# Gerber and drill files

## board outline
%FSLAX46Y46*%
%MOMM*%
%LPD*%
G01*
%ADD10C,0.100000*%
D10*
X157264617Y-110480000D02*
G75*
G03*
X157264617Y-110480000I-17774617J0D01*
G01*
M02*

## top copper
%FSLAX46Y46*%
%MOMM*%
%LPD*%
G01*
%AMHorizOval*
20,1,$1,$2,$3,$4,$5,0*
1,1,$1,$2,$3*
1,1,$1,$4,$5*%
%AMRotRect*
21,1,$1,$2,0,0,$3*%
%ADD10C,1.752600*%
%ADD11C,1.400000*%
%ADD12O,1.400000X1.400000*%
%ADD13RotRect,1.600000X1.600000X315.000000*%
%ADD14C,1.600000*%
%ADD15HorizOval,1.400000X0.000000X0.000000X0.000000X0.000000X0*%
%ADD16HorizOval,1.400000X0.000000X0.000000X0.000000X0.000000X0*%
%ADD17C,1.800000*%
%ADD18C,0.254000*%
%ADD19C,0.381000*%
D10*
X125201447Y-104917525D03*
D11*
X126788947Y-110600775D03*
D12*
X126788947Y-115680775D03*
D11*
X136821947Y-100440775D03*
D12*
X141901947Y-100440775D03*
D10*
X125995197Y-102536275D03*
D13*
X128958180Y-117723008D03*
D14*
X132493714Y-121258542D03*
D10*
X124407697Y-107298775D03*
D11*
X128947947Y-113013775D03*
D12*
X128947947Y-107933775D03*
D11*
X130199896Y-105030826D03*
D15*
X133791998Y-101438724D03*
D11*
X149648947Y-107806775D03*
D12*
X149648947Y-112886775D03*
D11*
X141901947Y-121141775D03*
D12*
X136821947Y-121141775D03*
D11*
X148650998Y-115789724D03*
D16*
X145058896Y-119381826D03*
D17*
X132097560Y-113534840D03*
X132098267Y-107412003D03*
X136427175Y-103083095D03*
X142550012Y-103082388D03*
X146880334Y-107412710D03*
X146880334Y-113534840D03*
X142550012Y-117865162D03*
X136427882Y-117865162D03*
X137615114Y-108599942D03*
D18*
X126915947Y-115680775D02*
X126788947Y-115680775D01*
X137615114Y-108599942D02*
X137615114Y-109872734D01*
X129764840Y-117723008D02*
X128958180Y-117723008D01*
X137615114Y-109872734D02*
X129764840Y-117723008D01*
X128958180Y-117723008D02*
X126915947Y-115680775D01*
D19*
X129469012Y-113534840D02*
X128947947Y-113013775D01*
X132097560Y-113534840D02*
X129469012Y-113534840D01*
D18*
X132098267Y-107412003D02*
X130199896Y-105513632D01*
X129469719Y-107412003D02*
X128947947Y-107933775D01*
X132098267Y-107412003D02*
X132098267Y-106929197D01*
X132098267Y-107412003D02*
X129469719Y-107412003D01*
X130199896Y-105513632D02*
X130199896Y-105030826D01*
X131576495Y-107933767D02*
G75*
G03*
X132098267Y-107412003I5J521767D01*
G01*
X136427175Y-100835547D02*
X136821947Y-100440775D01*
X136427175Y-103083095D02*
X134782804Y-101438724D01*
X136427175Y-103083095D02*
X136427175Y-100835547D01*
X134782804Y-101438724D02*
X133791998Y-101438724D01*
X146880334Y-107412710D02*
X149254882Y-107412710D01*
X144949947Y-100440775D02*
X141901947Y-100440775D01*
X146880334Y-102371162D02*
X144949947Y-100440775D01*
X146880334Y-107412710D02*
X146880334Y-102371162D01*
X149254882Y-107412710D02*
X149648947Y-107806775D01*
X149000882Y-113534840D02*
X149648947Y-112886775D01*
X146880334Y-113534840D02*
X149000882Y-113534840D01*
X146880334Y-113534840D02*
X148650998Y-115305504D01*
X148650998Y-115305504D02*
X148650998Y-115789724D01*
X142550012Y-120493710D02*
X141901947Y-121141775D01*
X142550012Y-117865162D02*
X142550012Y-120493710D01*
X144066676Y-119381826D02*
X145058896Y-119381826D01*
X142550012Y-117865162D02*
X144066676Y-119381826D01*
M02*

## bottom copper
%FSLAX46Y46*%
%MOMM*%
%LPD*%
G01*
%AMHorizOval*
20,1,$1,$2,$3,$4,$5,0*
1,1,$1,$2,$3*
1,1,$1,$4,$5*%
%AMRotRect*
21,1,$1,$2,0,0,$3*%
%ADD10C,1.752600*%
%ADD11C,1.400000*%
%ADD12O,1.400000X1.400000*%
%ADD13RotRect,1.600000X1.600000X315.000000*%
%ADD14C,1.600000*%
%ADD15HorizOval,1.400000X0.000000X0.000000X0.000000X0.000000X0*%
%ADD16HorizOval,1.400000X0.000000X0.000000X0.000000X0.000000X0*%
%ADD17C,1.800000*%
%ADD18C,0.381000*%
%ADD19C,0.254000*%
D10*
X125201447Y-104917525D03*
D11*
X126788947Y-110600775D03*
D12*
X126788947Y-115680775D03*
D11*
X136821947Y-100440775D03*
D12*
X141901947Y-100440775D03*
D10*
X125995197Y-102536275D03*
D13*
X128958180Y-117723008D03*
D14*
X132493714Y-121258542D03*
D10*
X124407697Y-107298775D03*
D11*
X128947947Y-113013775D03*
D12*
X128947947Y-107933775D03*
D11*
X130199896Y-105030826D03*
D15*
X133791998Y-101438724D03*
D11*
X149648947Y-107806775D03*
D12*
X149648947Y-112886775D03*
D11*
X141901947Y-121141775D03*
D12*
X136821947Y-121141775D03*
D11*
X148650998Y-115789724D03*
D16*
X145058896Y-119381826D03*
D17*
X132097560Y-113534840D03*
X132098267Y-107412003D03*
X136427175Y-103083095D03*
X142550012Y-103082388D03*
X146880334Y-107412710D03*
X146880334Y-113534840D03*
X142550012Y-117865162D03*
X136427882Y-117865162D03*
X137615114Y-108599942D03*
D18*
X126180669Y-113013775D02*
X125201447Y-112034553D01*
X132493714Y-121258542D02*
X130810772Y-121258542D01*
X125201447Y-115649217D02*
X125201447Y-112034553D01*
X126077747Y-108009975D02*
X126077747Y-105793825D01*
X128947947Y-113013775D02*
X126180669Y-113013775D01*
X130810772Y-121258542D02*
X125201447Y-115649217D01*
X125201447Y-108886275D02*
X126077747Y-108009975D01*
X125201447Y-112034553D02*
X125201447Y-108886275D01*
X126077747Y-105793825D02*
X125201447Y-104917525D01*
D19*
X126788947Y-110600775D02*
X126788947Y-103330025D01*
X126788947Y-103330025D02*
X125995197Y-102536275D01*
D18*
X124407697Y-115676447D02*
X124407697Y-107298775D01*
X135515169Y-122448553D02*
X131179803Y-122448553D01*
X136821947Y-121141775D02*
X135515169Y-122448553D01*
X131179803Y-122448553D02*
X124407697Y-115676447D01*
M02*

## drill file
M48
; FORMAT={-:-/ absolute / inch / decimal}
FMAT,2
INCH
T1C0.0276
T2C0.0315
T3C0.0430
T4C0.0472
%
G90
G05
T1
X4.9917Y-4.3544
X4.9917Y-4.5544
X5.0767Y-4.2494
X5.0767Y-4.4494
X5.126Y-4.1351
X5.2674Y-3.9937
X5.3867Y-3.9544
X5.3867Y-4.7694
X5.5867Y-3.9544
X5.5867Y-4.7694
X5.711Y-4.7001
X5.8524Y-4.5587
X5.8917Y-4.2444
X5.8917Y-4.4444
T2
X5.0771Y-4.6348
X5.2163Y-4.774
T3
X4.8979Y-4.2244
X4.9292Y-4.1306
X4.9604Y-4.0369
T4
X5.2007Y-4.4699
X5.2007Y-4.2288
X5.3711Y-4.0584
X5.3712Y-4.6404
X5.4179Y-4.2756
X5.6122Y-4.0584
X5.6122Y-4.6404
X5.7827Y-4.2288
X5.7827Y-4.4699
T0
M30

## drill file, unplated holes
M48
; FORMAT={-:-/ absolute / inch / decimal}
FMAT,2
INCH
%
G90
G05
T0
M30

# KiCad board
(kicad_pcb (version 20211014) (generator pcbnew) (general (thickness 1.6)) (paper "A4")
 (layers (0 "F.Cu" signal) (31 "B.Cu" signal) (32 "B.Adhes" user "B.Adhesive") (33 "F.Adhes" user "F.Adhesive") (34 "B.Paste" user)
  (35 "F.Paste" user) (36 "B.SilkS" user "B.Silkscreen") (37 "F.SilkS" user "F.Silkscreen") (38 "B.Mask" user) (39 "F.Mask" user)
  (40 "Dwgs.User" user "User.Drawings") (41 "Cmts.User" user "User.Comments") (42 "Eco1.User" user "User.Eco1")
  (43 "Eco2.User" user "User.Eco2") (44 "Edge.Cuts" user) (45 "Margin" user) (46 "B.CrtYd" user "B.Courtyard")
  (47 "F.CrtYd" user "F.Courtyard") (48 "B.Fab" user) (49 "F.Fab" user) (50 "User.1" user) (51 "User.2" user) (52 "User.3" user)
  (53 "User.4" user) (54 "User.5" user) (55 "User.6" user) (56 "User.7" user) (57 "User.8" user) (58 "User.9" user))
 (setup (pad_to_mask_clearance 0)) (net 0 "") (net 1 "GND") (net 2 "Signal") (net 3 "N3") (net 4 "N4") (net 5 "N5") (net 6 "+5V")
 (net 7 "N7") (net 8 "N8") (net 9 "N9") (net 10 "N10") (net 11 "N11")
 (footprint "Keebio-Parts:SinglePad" (layer "F.Cu") (at 125.201447 104.917525)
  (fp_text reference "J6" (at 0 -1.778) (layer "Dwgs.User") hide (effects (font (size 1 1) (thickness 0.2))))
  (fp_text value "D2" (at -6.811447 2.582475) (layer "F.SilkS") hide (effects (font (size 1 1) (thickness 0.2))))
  (pad "1" thru_hole circle locked (at 0 0 270) (size 1.7526 1.7526) (drill 1.0922) (layers *.Cu *.SilkS *.Mask) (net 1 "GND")))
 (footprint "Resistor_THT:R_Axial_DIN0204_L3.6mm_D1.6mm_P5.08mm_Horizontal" (layer "F.Cu") (at 126.788947 110.600775 -90)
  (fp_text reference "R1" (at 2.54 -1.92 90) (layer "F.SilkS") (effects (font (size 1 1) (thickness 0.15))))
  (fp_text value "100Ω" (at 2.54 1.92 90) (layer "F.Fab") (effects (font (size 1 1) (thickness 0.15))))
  (pad "1" thru_hole circle (at 0 0 270) (size 1.4 1.4) (drill 0.7) (layers *.Cu *.Mask) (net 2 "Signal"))
  (pad "2" thru_hole oval (at 5.08 0 270) (size 1.4 1.4) (drill 0.7) (layers *.Cu *.Mask) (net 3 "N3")))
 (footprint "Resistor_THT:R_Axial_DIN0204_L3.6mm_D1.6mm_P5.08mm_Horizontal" (layer "F.Cu") (at 136.821947 100.440775)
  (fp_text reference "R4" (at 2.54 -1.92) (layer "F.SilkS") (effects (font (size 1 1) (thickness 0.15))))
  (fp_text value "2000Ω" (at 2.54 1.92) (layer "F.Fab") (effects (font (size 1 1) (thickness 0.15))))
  (pad "1" thru_hole circle (at 0 0) (size 1.4 1.4) (drill 0.7) (layers *.Cu *.Mask) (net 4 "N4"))
  (pad "2" thru_hole oval (at 5.08 0) (size 1.4 1.4) (drill 0.7) (layers *.Cu *.Mask) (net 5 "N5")))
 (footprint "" (layer "F.Cu") (at 125.995197 102.536275)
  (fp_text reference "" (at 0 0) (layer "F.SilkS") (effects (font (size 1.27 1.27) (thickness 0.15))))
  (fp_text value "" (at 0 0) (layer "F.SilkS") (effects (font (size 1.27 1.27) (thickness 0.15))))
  (pad "1" thru_hole circle locked (at 0 0 270) (size 1.7526 1.7526) (drill 1.0922) (layers *.Cu *.SilkS *.Mask) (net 2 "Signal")))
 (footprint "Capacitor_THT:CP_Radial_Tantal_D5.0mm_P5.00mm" (layer "F.Cu") (at 128.95818 117.723008 -45)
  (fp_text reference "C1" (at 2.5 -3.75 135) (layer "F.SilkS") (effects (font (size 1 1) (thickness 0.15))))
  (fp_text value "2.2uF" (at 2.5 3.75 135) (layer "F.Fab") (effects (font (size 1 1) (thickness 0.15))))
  (pad "1" thru_hole rect (at 0 0 315) (size 1.6 1.6) (drill 0.8) (layers *.Cu *.Mask) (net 3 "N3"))
  (pad "2" thru_hole circle (at 5 0 315) (size 1.6 1.6) (drill 0.8) (layers *.Cu *.Mask) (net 1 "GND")))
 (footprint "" (layer "F.Cu") (at 124.407697 107.298775)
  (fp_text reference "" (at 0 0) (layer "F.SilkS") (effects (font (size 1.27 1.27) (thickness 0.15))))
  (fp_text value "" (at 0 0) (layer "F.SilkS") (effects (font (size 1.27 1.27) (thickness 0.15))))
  (pad "1" thru_hole circle locked (at 0 0 270) (size 1.7526 1.7526) (drill 1.0922) (layers *.Cu *.SilkS *.Mask) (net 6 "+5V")))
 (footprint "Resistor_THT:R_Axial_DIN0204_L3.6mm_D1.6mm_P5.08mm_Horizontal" (layer "F.Cu") (at 128.947947 113.013775 90)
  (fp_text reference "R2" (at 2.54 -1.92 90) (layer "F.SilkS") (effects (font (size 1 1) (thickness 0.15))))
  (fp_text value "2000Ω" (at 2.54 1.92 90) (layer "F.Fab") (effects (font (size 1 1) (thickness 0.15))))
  (pad "1" thru_hole circle (at 0 0 90) (size 1.4 1.4) (drill 0.7) (layers *.Cu *.Mask) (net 1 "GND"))
  (pad "2" thru_hole oval (at 5.08 0 90) (size 1.4 1.4) (drill 0.7) (layers *.Cu *.Mask) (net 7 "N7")))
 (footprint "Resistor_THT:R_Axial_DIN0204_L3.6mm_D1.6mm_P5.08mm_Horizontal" (layer "F.Cu") (at 130.199896 105.030826 45)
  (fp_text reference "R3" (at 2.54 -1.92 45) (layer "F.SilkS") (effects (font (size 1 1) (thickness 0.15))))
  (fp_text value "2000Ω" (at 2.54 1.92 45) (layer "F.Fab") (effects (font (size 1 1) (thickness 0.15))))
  (pad "1" thru_hole circle (at 0 0 45) (size 1.4 1.4) (drill 0.7) (layers *.Cu *.Mask) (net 7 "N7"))
  (pad "2" thru_hole oval (at 5.08 0 45) (size 1.4 1.4) (drill 0.7) (layers *.Cu *.Mask) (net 4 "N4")))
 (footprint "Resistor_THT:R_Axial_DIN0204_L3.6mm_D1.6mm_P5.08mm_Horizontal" (layer "F.Cu") (at 149.648947 107.806775 -90)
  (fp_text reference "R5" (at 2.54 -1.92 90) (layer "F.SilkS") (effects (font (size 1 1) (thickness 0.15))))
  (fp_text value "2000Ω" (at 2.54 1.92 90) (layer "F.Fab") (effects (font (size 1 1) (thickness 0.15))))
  (pad "1" thru_hole circle (at 0 0 270) (size 1.4 1.4) (drill 0.7) (layers *.Cu *.Mask) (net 5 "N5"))
  (pad "2" thru_hole oval (at 5.08 0 270) (size 1.4 1.4) (drill 0.7) (layers *.Cu *.Mask) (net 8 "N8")))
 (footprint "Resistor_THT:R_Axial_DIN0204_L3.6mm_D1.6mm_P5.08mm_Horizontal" (layer "F.Cu") (at 141.901947 121.141775 180)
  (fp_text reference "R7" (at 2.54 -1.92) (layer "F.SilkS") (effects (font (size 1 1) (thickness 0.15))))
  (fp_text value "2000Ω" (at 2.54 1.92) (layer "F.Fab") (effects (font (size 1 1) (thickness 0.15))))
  (pad "1" thru_hole circle (at 0 0 180) (size 1.4 1.4) (drill 0.7) (layers *.Cu *.Mask) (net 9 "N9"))
  (pad "2" thru_hole oval (at 5.08 0 180) (size 1.4 1.4) (drill 0.7) (layers *.Cu *.Mask) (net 6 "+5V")))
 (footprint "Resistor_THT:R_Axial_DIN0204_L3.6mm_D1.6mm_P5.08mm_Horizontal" (layer "F.Cu") (at 148.650998 115.789724 -135)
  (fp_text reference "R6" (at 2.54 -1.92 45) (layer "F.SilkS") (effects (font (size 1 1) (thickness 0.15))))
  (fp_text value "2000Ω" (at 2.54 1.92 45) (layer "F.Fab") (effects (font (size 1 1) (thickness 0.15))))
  (pad "1" thru_hole circle (at 0 0 225) (size 1.4 1.4) (drill 0.7) (layers *.Cu *.Mask) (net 8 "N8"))
  (pad "2" thru_hole oval (at 5.08 0 225) (size 1.4 1.4) (drill 0.7) (layers *.Cu *.Mask) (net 9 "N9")))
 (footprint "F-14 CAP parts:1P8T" (layer "B.Cu") (at 139.488947 110.473775 135)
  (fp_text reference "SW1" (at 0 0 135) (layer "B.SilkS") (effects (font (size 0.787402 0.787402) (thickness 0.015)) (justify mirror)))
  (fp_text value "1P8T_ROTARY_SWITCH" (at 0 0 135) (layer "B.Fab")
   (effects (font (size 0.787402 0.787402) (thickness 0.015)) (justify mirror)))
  (pad "1" thru_hole circle (at 3.062 -7.391 135) (size 1.8 1.8) (drill 1.2) (layers *.Cu *.Mask) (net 1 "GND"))
  (pad "2" thru_hole circle (at 7.391 -3.061 135) (size 1.8 1.8) (drill 1.2) (layers *.Cu *.Mask) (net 7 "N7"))
  (pad "3" thru_hole circle (at 7.391 3.061 135) (size 1.8 1.8) (drill 1.2) (layers *.Cu *.Mask) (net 4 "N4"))
  (pad "4" thru_hole circle (at 3.062 7.391 135) (size 1.8 1.8) (drill 1.2) (layers *.Cu *.Mask) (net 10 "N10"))
  (pad "5" thru_hole circle (at -3.062 7.391 135) (size 1.8 1.8) (drill 1.2) (layers *.Cu *.Mask) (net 5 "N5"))
  (pad "6" thru_hole circle (at -7.391 3.062 135) (size 1.8 1.8) (drill 1.2) (layers *.Cu *.Mask) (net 8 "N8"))
  (pad "7" thru_hole circle (at -7.391 -3.062 135) (size 1.8 1.8) (drill 1.2) (layers *.Cu *.Mask) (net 9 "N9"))
  (pad "8" thru_hole circle (at -3.062 -7.391 135) (size 1.8 1.8) (drill 1.2) (layers *.Cu *.Mask) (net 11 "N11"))
  (pad "9" thru_hole circle (at 2.65 0 135) (size 1.8 1.8) (drill 1.2) (layers *.Cu *.Mask) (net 3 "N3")))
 (gr_circle (center 139.49 110.48) (end 146.32 94.07) (layer "Edge.Cuts") (width 0.1) (fill none))
 (segment (start 126.915947 115.680775) (end 126.788947 115.680775) (width 0.254) (layer "F.Cu") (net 3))
 (segment (start 137.615114 108.599942) (end 137.615114 109.872734) (width 0.254) (layer "F.Cu") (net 3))
 (segment (start 129.76484 117.723008) (end 128.95818 117.723008) (width 0.254) (layer "F.Cu") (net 3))
 (segment (start 137.615114 109.872734) (end 129.76484 117.723008) (width 0.254) (layer "F.Cu") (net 3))
 (segment (start 128.95818 117.723008) (end 126.915947 115.680775) (width 0.254) (layer "F.Cu") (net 3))
 (segment (start 129.469012 113.53484) (end 128.947947 113.013775) (width 0.381) (layer "F.Cu") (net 1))
 (segment (start 132.09756 113.53484) (end 129.469012 113.53484) (width 0.381) (layer "F.Cu") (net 1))
 (segment (start 126.180669 113.013775) (end 125.201447 112.034553) (width 0.381) (layer "B.Cu") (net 1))
 (segment (start 132.493714 121.258542) (end 130.810772 121.258542) (width 0.381) (layer "B.Cu") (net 1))
 (segment (start 125.201447 115.649217) (end 125.201447 112.034553) (width 0.381) (layer "B.Cu") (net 1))
 (segment (start 126.077747 108.009975) (end 126.077747 105.793825) (width 0.381) (layer "B.Cu") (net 1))
 (segment (start 128.947947 113.013775) (end 126.180669 113.013775) (width 0.381) (layer "B.Cu") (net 1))
 (segment (start 130.810772 121.258542) (end 125.201447 115.649217) (width 0.381) (layer "B.Cu") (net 1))
 (segment (start 125.201447 108.886275) (end 126.077747 108.009975) (width 0.381) (layer "B.Cu") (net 1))
 (segment (start 125.201447 112.034553) (end 125.201447 108.886275) (width 0.381) (layer "B.Cu") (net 1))
 (segment (start 126.077747 105.793825) (end 125.201447 104.917525) (width 0.381) (layer "B.Cu") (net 1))
 (segment (start 126.788947 110.600775) (end 126.788947 103.330025) (width 0.254) (layer "B.Cu") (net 2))
 (segment (start 126.788947 103.330025) (end 125.995197 102.536275) (width 0.254) (layer "B.Cu") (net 2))
 (segment (start 132.098267 107.412003) (end 130.199896 105.513632) (width 0.254) (layer "F.Cu") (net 7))
 (segment (start 129.469719 107.412003) (end 128.947947 107.933775) (width 0.254) (layer "F.Cu") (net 7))
 (segment (start 132.098267 107.412003) (end 132.098267 106.929197) (width 0.254) (layer "F.Cu") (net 7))
 (segment (start 132.098267 107.412003) (end 129.469719 107.412003) (width 0.254) (layer "F.Cu") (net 7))
 (segment (start 130.199896 105.513632) (end 130.199896 105.030826) (width 0.254) (layer "F.Cu") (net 7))
 (arc (start 132.098267 107.412003) (mid 131.945444 107.780952) (end 131.576495 107.933775) (width 0.254) (layer "F.Cu") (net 7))
 (segment (start 136.427175 100.835547) (end 136.821947 100.440775) (width 0.254) (layer "F.Cu") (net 4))
 (segment (start 136.427175 103.083095) (end 134.782804 101.438724) (width 0.254) (layer "F.Cu") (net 4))
 (segment (start 136.427175 103.083095) (end 136.427175 100.835547) (width 0.254) (layer "F.Cu") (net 4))
 (segment (start 134.782804 101.438724) (end 133.791998 101.438724) (width 0.254) (layer "F.Cu") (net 4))
 (segment (start 146.880334 107.41271) (end 149.254882 107.41271) (width 0.254) (layer "F.Cu") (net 5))
 (segment (start 144.949947 100.440775) (end 141.901947 100.440775) (width 0.254) (layer "F.Cu") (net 5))
 (segment (start 146.880334 102.371162) (end 144.949947 100.440775) (width 0.254) (layer "F.Cu") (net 5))
 (segment (start 146.880334 107.41271) (end 146.880334 102.371162) (width 0.254) (layer "F.Cu") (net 5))
 (segment (start 149.254882 107.41271) (end 149.648947 107.806775) (width 0.254) (layer "F.Cu") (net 5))
 (segment (start 149.000882 113.53484) (end 149.648947 112.886775) (width 0.254) (layer "F.Cu") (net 8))
 (segment (start 146.880334 113.53484) (end 149.000882 113.53484) (width 0.254) (layer "F.Cu") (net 8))
 (segment (start 146.880334 113.53484) (end 148.650998 115.305504) (width 0.254) (layer "F.Cu") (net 8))
 (segment (start 148.650998 115.305504) (end 148.650998 115.789724) (width 0.254) (layer "F.Cu") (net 8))
 (segment (start 142.550012 120.49371) (end 141.901947 121.141775) (width 0.254) (layer "F.Cu") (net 9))
 (segment (start 142.550012 117.865162) (end 142.550012 120.49371) (width 0.254) (layer "F.Cu") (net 9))
 (segment (start 144.066676 119.381826) (end 145.058896 119.381826) (width 0.254) (layer "F.Cu") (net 9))
 (segment (start 142.550012 117.865162) (end 144.066676 119.381826) (width 0.254) (layer "F.Cu") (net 9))
 (segment (start 124.407697 115.676447) (end 124.407697 107.298775) (width 0.381) (layer "B.Cu") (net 6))
 (segment (start 135.515169 122.448553) (end 131.179803 122.448553) (width 0.381) (layer "B.Cu") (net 6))
 (segment (start 136.821947 121.141775) (end 135.515169 122.448553) (width 0.381) (layer "B.Cu") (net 6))
 (segment (start 131.179803 122.448553) (end 124.407697 115.676447) (width 0.381) (layer "B.Cu") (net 6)))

